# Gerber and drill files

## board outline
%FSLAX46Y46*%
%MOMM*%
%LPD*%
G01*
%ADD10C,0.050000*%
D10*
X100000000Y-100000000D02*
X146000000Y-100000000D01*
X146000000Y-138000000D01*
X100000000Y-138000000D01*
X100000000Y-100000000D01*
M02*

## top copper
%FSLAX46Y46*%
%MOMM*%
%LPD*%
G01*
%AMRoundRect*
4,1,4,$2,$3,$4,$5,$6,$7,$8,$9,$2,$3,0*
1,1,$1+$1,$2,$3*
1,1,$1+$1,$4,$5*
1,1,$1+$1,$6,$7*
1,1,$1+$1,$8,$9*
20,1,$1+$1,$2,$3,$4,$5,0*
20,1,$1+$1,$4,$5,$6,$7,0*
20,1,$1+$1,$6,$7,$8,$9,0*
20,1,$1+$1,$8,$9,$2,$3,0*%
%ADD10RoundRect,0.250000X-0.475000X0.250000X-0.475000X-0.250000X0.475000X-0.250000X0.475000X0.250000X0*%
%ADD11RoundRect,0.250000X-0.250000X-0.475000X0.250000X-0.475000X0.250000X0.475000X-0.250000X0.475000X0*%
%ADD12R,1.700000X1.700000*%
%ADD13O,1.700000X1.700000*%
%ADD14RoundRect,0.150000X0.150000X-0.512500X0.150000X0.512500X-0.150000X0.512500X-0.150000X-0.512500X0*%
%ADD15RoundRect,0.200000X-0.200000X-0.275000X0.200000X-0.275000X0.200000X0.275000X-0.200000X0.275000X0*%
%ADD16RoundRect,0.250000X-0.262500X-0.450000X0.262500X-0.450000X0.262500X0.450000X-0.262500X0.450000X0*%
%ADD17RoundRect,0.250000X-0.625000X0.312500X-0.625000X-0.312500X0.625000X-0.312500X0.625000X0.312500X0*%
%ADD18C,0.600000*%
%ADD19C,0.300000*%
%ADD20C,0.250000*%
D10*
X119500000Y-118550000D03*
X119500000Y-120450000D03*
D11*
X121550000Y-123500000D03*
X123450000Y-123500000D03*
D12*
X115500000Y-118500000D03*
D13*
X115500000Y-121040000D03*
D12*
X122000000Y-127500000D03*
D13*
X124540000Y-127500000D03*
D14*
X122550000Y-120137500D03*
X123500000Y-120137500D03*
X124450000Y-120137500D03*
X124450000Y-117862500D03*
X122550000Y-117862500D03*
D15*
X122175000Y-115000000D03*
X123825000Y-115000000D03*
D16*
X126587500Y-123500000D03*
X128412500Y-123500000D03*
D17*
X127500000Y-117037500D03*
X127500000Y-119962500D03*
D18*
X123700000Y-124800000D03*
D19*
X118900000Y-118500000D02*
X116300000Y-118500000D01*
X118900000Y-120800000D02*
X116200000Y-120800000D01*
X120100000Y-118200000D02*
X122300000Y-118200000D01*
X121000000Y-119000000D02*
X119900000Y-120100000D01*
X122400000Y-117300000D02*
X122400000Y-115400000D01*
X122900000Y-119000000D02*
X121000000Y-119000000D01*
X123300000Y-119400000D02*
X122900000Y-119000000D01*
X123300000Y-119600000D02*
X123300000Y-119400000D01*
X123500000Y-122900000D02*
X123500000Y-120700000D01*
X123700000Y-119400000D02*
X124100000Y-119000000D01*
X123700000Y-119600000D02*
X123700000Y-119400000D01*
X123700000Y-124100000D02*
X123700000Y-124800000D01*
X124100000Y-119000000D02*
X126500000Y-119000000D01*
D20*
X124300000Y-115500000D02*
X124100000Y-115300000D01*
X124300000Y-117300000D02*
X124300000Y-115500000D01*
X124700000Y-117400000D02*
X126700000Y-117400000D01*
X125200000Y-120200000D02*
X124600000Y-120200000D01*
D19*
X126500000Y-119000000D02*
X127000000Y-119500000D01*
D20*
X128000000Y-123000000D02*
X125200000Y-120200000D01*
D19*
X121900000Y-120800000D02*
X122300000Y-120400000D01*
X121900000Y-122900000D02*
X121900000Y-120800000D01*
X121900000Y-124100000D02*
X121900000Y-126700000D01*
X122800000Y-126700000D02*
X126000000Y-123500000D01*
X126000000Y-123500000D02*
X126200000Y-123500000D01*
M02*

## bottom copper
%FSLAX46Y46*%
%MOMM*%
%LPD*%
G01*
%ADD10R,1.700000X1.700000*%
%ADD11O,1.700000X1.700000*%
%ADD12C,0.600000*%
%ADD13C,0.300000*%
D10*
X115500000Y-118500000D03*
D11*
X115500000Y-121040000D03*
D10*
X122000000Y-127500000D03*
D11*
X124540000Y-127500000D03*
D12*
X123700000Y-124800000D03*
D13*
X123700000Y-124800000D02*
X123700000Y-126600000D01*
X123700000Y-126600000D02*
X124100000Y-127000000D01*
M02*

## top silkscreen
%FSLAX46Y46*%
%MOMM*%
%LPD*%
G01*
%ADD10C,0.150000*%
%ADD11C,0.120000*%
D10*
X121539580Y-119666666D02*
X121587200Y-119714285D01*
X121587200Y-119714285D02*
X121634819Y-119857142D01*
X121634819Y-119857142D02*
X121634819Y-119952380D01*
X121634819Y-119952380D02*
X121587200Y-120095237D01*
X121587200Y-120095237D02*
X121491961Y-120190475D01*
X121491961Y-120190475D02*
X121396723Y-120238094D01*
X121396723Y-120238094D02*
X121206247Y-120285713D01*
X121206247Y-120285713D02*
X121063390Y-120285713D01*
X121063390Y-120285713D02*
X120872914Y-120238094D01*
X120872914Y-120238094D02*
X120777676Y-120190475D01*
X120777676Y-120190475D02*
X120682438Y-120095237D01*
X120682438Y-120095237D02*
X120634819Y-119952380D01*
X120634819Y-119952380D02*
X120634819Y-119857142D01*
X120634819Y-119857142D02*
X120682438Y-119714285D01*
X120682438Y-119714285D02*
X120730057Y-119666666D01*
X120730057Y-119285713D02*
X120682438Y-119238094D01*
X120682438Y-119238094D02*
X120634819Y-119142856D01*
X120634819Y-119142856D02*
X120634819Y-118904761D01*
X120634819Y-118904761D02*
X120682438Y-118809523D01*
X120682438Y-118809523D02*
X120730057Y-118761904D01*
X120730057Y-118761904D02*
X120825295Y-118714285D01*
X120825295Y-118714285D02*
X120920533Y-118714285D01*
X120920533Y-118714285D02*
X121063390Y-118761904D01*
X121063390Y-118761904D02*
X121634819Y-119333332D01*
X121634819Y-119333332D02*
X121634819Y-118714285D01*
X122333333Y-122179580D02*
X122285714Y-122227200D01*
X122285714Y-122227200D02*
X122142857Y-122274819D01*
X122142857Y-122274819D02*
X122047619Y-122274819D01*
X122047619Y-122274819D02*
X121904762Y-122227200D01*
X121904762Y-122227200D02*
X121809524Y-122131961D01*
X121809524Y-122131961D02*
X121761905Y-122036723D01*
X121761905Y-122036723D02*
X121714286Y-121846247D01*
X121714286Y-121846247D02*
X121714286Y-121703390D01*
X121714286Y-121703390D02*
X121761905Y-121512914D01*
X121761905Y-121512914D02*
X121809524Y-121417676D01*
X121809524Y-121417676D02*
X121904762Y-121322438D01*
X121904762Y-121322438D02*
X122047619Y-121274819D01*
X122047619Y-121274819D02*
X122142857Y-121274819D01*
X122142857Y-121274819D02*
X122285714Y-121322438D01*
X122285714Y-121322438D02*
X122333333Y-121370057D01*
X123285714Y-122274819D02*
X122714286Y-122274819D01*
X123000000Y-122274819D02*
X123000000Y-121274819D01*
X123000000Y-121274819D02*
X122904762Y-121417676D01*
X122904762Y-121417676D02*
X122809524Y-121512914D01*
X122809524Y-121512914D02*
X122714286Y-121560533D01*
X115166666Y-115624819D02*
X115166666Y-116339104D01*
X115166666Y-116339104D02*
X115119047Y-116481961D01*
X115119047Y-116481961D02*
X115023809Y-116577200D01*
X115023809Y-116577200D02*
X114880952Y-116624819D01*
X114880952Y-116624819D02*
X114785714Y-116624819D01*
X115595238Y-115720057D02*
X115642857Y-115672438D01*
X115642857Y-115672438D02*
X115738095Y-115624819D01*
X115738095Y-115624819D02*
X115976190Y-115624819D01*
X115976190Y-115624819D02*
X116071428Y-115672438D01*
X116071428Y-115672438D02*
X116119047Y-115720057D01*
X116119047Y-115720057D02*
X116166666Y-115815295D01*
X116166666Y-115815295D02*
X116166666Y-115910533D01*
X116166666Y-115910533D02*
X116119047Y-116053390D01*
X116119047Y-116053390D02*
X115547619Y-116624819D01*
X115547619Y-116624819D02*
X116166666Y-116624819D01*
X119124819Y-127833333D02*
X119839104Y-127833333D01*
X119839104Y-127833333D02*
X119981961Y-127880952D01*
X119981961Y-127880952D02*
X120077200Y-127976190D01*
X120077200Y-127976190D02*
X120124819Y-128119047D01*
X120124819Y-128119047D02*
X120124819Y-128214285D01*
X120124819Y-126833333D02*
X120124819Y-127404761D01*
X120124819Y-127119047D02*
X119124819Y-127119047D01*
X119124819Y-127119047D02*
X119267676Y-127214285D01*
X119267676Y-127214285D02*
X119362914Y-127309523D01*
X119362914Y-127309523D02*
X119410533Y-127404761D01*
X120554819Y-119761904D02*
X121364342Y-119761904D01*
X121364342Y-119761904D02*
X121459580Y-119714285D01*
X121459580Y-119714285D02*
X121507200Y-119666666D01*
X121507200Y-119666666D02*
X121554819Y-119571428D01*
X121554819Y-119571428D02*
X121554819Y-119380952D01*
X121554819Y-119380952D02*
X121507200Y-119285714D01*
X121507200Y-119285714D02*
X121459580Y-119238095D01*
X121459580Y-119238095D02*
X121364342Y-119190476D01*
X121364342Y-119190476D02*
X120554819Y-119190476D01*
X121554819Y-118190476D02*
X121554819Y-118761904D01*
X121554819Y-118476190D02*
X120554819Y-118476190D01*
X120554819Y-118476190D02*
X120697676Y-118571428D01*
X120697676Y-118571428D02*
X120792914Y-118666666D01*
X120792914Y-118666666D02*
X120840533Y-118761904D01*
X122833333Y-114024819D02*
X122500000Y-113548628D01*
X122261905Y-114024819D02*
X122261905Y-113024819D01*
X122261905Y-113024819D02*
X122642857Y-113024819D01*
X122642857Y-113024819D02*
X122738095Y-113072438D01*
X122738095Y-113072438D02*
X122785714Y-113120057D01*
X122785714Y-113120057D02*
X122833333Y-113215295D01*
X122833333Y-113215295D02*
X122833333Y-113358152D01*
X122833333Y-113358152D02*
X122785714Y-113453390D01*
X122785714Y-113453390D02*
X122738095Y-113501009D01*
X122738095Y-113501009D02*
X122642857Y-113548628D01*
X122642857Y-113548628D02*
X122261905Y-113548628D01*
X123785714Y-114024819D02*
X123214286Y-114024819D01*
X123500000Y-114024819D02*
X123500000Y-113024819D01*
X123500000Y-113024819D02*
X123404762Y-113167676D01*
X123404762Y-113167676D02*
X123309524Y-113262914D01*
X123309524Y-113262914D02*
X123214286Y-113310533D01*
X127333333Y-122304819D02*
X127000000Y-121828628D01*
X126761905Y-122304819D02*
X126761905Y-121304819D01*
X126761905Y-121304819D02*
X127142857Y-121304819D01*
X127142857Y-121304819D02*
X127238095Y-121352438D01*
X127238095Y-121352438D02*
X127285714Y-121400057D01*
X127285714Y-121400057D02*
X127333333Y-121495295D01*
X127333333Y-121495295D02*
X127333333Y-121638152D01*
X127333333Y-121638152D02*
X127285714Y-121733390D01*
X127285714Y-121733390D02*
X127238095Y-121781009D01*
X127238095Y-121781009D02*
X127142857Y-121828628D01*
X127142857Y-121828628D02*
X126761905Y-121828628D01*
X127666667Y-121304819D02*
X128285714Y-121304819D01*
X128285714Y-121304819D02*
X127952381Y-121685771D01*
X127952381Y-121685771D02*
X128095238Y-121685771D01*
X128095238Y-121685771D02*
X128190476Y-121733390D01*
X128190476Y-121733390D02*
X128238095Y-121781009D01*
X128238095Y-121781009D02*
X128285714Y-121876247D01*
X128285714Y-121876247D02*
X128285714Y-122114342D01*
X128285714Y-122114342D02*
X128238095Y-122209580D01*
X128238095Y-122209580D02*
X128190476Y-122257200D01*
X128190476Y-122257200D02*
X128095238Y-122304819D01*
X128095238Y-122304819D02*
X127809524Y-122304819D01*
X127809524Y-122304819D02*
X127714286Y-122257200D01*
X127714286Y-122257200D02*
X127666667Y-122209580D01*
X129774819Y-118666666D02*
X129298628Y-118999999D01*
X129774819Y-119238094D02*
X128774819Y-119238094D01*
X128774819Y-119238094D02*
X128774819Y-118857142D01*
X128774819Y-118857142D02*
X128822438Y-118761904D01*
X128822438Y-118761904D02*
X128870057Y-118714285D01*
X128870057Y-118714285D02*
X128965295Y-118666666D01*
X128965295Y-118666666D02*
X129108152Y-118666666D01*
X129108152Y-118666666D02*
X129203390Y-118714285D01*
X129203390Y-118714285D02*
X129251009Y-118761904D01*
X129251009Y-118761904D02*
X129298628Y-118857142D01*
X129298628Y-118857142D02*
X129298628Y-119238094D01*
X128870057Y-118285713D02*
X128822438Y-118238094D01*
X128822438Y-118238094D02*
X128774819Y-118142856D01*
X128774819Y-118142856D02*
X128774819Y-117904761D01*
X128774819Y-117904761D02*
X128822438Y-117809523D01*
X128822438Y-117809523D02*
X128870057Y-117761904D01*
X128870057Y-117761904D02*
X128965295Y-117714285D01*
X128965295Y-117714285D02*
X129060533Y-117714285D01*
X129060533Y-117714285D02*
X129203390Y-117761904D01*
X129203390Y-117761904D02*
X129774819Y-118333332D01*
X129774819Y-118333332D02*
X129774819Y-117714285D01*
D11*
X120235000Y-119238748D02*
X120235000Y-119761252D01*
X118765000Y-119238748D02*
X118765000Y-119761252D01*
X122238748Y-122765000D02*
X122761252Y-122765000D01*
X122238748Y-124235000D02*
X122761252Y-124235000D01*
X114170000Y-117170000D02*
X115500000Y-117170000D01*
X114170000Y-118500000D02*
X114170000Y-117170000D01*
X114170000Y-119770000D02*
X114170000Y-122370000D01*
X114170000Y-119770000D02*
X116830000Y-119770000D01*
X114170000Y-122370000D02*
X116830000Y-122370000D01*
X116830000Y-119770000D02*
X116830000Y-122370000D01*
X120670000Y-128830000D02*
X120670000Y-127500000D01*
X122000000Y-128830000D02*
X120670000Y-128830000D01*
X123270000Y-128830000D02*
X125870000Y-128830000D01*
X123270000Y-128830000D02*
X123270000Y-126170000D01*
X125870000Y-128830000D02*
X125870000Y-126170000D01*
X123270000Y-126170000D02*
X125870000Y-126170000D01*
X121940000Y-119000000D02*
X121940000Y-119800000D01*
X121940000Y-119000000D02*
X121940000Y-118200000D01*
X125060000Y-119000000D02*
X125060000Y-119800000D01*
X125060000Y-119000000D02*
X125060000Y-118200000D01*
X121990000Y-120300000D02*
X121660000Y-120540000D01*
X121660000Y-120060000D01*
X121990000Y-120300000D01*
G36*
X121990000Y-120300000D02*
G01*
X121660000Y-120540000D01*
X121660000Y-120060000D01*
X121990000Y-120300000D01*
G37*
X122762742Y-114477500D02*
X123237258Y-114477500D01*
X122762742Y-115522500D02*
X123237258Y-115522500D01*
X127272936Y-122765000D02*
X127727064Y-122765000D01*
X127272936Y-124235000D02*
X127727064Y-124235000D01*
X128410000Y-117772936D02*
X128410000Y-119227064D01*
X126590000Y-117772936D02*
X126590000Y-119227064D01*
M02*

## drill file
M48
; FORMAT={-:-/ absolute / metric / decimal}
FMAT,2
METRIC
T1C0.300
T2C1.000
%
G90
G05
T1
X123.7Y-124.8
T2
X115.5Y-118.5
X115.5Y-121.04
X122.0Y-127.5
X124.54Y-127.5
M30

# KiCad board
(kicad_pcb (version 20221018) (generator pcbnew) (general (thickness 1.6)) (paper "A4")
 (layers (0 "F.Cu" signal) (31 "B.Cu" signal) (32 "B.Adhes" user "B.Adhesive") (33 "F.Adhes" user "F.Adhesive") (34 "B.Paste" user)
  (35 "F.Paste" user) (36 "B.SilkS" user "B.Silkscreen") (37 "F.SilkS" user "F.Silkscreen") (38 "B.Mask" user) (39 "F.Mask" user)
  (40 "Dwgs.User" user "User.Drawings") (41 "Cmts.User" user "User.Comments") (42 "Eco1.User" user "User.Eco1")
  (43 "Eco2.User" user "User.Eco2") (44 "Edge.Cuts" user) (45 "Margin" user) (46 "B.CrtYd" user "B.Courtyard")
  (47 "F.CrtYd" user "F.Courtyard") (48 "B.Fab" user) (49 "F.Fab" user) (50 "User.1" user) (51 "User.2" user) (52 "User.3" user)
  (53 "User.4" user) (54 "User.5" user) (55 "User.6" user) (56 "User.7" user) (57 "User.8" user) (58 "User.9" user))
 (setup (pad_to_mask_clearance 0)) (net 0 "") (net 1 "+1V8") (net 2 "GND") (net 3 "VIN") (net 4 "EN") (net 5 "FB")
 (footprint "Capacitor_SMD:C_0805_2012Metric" (layer "F.Cu") (at 119.5 119.5 -90)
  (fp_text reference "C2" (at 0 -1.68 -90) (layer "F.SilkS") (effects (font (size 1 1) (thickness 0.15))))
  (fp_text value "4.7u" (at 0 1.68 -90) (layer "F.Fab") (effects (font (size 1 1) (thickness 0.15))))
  (fp_line (start -0.261252 -0.735) (end 0.261252 -0.735) (stroke (width 0.12) (type solid)) (layer "F.SilkS"))
  (fp_line (start -0.261252 0.735) (end 0.261252 0.735) (stroke (width 0.12) (type solid)) (layer "F.SilkS"))
  (pad "1" smd roundrect (at -0.95 0 270) (size 1 1.45) (layers "F.Cu" "F.Paste" "F.Mask") (roundrect_rratio 0.25) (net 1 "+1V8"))
  (pad "2" smd roundrect (at 0.95 0 270) (size 1 1.45) (layers "F.Cu" "F.Paste" "F.Mask") (roundrect_rratio 0.25) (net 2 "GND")))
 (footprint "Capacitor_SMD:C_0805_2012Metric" (layer "F.Cu") (at 122.5 123.5)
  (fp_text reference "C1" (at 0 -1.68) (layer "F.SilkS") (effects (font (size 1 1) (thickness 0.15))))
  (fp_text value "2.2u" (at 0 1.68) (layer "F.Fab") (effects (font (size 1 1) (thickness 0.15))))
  (fp_line (start -0.261252 -0.735) (end 0.261252 -0.735) (stroke (width 0.12) (type solid)) (layer "F.SilkS"))
  (fp_line (start -0.261252 0.735) (end 0.261252 0.735) (stroke (width 0.12) (type solid)) (layer "F.SilkS"))
  (pad "1" smd roundrect (at -0.95 0) (size 1 1.45) (layers "F.Cu" "F.Paste" "F.Mask") (roundrect_rratio 0.25) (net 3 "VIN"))
  (pad "2" smd roundrect (at 0.95 0) (size 1 1.45) (layers "F.Cu" "F.Paste" "F.Mask") (roundrect_rratio 0.25) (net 2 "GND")))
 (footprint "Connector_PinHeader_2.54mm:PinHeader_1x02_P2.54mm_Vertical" (layer "F.Cu") (at 115.5 118.5)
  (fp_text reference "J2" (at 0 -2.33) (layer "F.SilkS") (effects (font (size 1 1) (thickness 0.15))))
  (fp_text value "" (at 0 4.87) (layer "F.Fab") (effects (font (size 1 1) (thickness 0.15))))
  (fp_line (start -1.33 -1.33) (end 0 -1.33) (stroke (width 0.12) (type solid)) (layer "F.SilkS"))
  (fp_line (start -1.33 0) (end -1.33 -1.33) (stroke (width 0.12) (type solid)) (layer "F.SilkS"))
  (fp_line (start -1.33 1.27) (end -1.33 3.87) (stroke (width 0.12) (type solid)) (layer "F.SilkS"))
  (fp_line (start -1.33 1.27) (end 1.33 1.27) (stroke (width 0.12) (type solid)) (layer "F.SilkS"))
  (fp_line (start -1.33 3.87) (end 1.33 3.87) (stroke (width 0.12) (type solid)) (layer "F.SilkS"))
  (fp_line (start 1.33 1.27) (end 1.33 3.87) (stroke (width 0.12) (type solid)) (layer "F.SilkS"))
  (pad "1" thru_hole rect (at 0 0) (size 1.7 1.7) (drill 1) (layers "*.Cu" "*.Mask") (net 1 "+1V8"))
  (pad "2" thru_hole oval (at 0 2.54) (size 1.7 1.7) (drill 1) (layers "*.Cu" "*.Mask") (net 2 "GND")))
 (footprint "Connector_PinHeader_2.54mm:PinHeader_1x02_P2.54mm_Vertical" (layer "F.Cu") (at 122 127.5 90)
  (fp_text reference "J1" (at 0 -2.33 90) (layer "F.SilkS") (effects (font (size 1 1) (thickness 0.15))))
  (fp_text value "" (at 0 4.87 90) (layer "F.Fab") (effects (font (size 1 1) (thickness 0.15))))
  (fp_line (start -1.33 -1.33) (end 0 -1.33) (stroke (width 0.12) (type solid)) (layer "F.SilkS"))
  (fp_line (start -1.33 0) (end -1.33 -1.33) (stroke (width 0.12) (type solid)) (layer "F.SilkS"))
  (fp_line (start -1.33 1.27) (end -1.33 3.87) (stroke (width 0.12) (type solid)) (layer "F.SilkS"))
  (fp_line (start -1.33 1.27) (end 1.33 1.27) (stroke (width 0.12) (type solid)) (layer "F.SilkS"))
  (fp_line (start -1.33 3.87) (end 1.33 3.87) (stroke (width 0.12) (type solid)) (layer "F.SilkS"))
  (fp_line (start 1.33 1.27) (end 1.33 3.87) (stroke (width 0.12) (type solid)) (layer "F.SilkS"))
  (pad "1" thru_hole rect (at 0 0 90) (size 1.7 1.7) (drill 1) (layers "*.Cu" "*.Mask") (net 3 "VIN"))
  (pad "2" thru_hole oval (at 0 2.54 90) (size 1.7 1.7) (drill 1) (layers "*.Cu" "*.Mask") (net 2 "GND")))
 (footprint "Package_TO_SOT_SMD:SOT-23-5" (layer "F.Cu") (at 123.5 119 90)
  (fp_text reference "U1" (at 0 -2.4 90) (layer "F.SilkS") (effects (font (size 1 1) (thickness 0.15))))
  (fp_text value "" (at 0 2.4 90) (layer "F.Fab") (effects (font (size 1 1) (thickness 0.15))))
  (fp_line (start 0 -1.56) (end -0.8 -1.56) (stroke (width 0.12) (type solid)) (layer "F.SilkS"))
  (fp_line (start 0 -1.56) (end 0.8 -1.56) (stroke (width 0.12) (type solid)) (layer "F.SilkS"))
  (fp_line (start 0 1.56) (end -0.8 1.56) (stroke (width 0.12) (type solid)) (layer "F.SilkS"))
  (fp_line (start 0 1.56) (end 0.8 1.56) (stroke (width 0.12) (type solid)) (layer "F.SilkS"))
  (fp_poly
   (pts (xy -1.3 -1.51) (xy -1.54 -1.84) (xy -1.06 -1.84) (xy -1.3 -1.51)) (stroke (width 0.12) (type solid)) (fill solid) (layer "F.SilkS"))
  (pad "1" smd roundrect (at -1.1375 -0.95 90) (size 1.325 0.6) (layers "F.Cu" "F.Paste" "F.Mask") (roundrect_rratio 0.25) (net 3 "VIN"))
  (pad "2" smd roundrect (at -1.1375 0 90) (size 1.325 0.6) (layers "F.Cu" "F.Paste" "F.Mask") (roundrect_rratio 0.25) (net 2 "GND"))
  (pad "3" smd roundrect (at -1.1375 0.95 90) (size 1.325 0.6) (layers "F.Cu" "F.Paste" "F.Mask") (roundrect_rratio 0.25) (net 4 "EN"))
  (pad "4" smd roundrect (at 1.1375 0.95 90) (size 1.325 0.6) (layers "F.Cu" "F.Paste" "F.Mask") (roundrect_rratio 0.25) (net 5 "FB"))
  (pad "5" smd roundrect (at 1.1375 -0.95 90) (size 1.325 0.6) (layers "F.Cu" "F.Paste" "F.Mask") (roundrect_rratio 0.25) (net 1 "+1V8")))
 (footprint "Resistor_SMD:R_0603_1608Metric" (layer "F.Cu") (at 123 115)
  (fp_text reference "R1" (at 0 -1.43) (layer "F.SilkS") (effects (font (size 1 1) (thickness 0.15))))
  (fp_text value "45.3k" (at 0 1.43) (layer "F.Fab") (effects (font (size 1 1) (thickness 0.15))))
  (fp_line (start -0.237258 -0.5225) (end 0.237258 -0.5225) (stroke (width 0.12) (type solid)) (layer "F.SilkS"))
  (fp_line (start -0.237258 0.5225) (end 0.237258 0.5225) (stroke (width 0.12) (type solid)) (layer "F.SilkS"))
  (pad "1" smd roundrect (at -0.825 0) (size 0.8 0.95) (layers "F.Cu" "F.Paste" "F.Mask") (roundrect_rratio 0.25) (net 1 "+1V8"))
  (pad "2" smd roundrect (at 0.825 0) (size 0.8 0.95) (layers "F.Cu" "F.Paste" "F.Mask") (roundrect_rratio 0.25) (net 5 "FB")))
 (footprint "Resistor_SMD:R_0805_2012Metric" (layer "F.Cu") (at 127.5 123.5)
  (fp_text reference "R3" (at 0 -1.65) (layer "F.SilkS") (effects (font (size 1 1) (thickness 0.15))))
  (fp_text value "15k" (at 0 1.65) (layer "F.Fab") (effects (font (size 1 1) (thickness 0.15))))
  (fp_line (start -0.227064 -0.735) (end 0.227064 -0.735) (stroke (width 0.12) (type solid)) (layer "F.SilkS"))
  (fp_line (start -0.227064 0.735) (end 0.227064 0.735) (stroke (width 0.12) (type solid)) (layer "F.SilkS"))
  (pad "1" smd roundrect (at -0.9125 0) (size 1.025 1.4) (layers "F.Cu" "F.Paste" "F.Mask") (roundrect_rratio 0.243902) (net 3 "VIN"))
  (pad "2" smd roundrect (at 0.9125 0) (size 1.025 1.4) (layers "F.Cu" "F.Paste" "F.Mask") (roundrect_rratio 0.243902) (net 4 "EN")))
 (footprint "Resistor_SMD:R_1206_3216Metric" (layer "F.Cu") (at 127.5 118.5 -90)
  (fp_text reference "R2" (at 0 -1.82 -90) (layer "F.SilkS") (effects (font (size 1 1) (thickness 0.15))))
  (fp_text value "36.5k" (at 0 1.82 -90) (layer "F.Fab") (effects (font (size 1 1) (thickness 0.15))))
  (fp_line (start -0.727064 -0.91) (end 0.727064 -0.91) (stroke (width 0.12) (type solid)) (layer "F.SilkS"))
  (fp_line (start -0.727064 0.91) (end 0.727064 0.91) (stroke (width 0.12) (type solid)) (layer "F.SilkS"))
  (pad "1" smd roundrect (at -1.4625 0 270) (size 1.125 1.75) (layers "F.Cu" "F.Paste" "F.Mask") (roundrect_rratio 0.222222) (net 5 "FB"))
  (pad "2" smd roundrect (at 1.4625 0 270) (size 1.125 1.75) (layers "F.Cu" "F.Paste" "F.Mask") (roundrect_rratio 0.222222) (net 2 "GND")))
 (gr_rect (start 100 100) (end 146 138) (stroke (width 0.05) (type default)) (fill none) (layer "Edge.Cuts"))
 (segment (start 118.9 118.5) (end 116.3 118.5) (width 0.3) (layer "F.Cu") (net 1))
 (segment (start 118.9 120.8) (end 116.2 120.8) (width 0.3) (layer "F.Cu") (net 2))
 (segment (start 120.1 118.2) (end 122.3 118.2) (width 0.3) (layer "F.Cu") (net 1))
 (segment (start 121 119) (end 119.9 120.1) (width 0.3) (layer "F.Cu") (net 2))
 (segment (start 122.4 117.3) (end 122.4 115.4) (width 0.3) (layer "F.Cu") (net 1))
 (segment (start 122.9 119) (end 121 119) (width 0.3) (layer "F.Cu") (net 2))
 (segment (start 123.3 119.4) (end 122.9 119) (width 0.3) (layer "F.Cu") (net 2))
 (segment (start 123.3 119.6) (end 123.3 119.4) (width 0.3) (layer "F.Cu") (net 2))
 (segment (start 123.5 122.9) (end 123.5 120.7) (width 0.3) (layer "F.Cu") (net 2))
 (segment (start 123.7 119.4) (end 124.1 119) (width 0.3) (layer "F.Cu") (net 2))
 (segment (start 123.7 119.6) (end 123.7 119.4) (width 0.3) (layer "F.Cu") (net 2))
 (segment (start 123.7 124.1) (end 123.7 124.8) (width 0.3) (layer "F.Cu") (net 2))
 (segment (start 124.1 119) (end 126.5 119) (width 0.3) (layer "F.Cu") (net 2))
 (segment (start 124.3 115.5) (end 124.1 115.3) (width 0.25) (layer "F.Cu") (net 5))
 (segment (start 124.3 117.3) (end 124.3 115.5) (width 0.25) (layer "F.Cu") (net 5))
 (segment (start 124.7 117.4) (end 126.7 117.4) (width 0.25) (layer "F.Cu") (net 5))
 (segment (start 125.2 120.2) (end 124.6 120.2) (width 0.25) (layer "F.Cu") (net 4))
 (segment (start 126.5 119) (end 127 119.5) (width 0.3) (layer "F.Cu") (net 2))
 (segment (start 128 123) (end 125.2 120.2) (width 0.25) (layer "F.Cu") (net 4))
 (via (at 123.7 124.8) (size 0.6) (drill 0.3) (layers "F.Cu" "B.Cu") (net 2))
 (segment (start 121.9 120.8) (end 122.3 120.4) (width 0.3) (layer "F.Cu") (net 3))
 (segment (start 121.9 122.9) (end 121.9 120.8) (width 0.3) (layer "F.Cu") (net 3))
 (segment (start 121.9 124.1) (end 121.9 126.7) (width 0.3) (layer "F.Cu") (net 3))
 (segment (start 122.8 126.7) (end 126 123.5) (width 0.3) (layer "F.Cu") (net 3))
 (segment (start 123.7 124.8) (end 123.7 126.6) (width 0.3) (layer "B.Cu") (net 2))
 (segment (start 123.7 126.6) (end 124.1 127) (width 0.3) (layer "B.Cu") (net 2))
 (segment (start 126 123.5) (end 126.2 123.5) (width 0.3) (layer "F.Cu") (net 3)))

